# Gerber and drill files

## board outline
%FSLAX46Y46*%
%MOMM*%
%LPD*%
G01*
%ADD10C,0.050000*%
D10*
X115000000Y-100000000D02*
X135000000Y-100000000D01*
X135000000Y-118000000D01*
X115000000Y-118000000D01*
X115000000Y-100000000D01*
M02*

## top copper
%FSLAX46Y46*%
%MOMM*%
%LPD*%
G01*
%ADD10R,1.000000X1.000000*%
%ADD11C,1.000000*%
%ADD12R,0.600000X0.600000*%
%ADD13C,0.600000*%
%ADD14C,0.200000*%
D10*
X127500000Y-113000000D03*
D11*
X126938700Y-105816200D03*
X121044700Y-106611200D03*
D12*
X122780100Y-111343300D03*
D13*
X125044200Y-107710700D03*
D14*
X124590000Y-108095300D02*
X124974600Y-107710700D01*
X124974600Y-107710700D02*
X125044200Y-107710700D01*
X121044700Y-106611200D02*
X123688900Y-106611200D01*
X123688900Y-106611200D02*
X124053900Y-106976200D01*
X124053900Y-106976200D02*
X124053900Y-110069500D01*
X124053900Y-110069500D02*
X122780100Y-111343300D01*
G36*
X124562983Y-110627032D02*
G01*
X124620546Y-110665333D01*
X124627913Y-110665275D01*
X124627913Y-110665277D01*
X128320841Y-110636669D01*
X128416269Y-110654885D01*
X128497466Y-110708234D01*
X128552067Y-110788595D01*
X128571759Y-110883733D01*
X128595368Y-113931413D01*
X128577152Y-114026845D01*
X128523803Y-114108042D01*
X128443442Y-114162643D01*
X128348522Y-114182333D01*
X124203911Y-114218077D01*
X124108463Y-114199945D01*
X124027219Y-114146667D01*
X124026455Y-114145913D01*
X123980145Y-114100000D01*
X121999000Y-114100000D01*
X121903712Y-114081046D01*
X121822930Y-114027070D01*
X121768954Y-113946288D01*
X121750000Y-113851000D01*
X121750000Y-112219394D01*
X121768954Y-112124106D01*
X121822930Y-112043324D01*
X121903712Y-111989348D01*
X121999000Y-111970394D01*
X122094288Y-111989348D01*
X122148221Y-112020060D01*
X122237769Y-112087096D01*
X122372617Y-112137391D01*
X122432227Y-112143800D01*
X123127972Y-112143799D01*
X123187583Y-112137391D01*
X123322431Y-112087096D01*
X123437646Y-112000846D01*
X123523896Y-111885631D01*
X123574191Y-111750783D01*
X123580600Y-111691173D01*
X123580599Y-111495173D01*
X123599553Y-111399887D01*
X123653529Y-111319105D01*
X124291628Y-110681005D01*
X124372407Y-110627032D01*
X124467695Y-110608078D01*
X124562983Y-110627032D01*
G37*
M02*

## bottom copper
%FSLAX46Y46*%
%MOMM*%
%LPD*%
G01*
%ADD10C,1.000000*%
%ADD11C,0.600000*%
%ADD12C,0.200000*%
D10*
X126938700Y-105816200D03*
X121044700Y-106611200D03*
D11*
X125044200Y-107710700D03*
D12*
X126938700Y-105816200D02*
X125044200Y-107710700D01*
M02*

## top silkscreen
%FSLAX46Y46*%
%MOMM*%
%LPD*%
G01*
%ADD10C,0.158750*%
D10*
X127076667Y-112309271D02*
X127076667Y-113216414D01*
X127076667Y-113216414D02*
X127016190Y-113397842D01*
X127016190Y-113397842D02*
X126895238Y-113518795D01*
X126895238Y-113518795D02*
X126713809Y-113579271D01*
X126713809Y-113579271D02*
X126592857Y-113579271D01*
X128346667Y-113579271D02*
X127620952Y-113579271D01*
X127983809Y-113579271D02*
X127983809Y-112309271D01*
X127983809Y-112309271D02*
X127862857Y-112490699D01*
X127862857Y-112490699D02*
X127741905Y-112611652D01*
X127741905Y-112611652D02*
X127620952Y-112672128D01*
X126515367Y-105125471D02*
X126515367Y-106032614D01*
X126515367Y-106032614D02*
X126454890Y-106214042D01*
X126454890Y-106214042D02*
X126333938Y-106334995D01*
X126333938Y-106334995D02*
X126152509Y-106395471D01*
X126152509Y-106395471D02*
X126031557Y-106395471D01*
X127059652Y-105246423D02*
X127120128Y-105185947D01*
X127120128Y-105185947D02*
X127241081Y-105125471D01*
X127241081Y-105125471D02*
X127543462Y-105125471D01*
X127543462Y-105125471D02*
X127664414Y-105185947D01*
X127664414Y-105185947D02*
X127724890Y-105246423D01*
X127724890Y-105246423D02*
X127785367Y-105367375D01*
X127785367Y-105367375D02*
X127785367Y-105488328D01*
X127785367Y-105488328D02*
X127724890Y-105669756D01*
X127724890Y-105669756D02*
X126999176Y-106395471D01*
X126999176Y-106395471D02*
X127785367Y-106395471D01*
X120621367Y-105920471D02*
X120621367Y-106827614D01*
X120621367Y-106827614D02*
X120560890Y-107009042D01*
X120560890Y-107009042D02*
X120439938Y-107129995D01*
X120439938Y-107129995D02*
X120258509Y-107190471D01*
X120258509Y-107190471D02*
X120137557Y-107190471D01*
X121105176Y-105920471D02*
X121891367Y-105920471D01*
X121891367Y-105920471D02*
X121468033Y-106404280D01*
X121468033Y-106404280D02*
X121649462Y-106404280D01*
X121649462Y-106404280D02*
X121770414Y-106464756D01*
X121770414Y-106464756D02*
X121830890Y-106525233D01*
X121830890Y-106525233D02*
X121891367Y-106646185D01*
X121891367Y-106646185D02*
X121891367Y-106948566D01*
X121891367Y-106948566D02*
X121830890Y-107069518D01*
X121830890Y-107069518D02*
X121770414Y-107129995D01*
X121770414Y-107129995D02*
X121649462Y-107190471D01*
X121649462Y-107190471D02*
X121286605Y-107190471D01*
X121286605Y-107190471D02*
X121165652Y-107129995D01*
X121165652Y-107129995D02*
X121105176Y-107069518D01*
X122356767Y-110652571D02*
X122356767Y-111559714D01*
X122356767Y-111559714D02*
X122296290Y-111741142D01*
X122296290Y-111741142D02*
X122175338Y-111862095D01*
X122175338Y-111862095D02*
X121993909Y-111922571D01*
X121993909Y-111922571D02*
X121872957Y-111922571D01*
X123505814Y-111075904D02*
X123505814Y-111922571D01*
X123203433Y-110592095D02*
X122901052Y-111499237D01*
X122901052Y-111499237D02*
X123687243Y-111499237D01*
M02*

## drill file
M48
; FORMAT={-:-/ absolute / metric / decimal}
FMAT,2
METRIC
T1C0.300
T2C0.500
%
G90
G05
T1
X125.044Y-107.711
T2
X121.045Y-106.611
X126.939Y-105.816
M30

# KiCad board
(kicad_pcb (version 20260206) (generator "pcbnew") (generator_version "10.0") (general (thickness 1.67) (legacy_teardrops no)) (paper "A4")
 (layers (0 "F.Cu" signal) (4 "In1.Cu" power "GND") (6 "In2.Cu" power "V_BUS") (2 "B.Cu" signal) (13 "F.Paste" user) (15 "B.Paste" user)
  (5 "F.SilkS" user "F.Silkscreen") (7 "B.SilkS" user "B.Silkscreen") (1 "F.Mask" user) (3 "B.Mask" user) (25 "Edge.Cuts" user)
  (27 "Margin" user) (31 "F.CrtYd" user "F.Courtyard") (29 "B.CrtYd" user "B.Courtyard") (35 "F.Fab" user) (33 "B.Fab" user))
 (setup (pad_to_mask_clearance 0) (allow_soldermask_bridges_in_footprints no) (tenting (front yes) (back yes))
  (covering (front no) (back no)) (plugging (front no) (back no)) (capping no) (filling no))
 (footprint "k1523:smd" (layer "F.Cu") (at 127.5 113)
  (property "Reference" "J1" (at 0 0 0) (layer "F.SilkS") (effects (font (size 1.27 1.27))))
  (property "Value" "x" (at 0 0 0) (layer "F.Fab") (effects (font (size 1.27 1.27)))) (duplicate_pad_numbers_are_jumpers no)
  (pad "1" smd rect (at 0 0) (size 1 1) (layers "F.Cu" "F.Mask") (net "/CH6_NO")))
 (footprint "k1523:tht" (layer "F.Cu") (at 126.9387 105.8162)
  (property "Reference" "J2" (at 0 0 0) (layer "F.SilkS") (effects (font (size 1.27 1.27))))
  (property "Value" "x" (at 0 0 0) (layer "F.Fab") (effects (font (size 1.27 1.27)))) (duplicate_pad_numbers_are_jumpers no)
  (pad "1" thru_hole circle (at 0 0) (size 1 1) (drill 0.5) (layers "*.Cu" "*.Mask") (remove_unused_layers no) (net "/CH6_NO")))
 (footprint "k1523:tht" (layer "F.Cu") (at 121.0447 106.6112)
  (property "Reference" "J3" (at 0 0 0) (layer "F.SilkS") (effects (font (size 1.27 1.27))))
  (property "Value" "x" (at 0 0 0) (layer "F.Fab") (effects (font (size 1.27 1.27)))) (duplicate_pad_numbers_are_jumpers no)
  (pad "1" thru_hole circle (at 0 0) (size 1 1) (drill 0.5) (layers "*.Cu" "*.Mask") (remove_unused_layers no) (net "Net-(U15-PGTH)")))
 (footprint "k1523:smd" (layer "F.Cu") (at 122.7801 111.3433)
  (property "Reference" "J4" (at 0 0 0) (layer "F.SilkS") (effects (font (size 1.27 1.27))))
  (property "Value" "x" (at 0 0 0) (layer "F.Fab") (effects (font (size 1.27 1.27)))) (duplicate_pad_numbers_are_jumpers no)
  (pad "1" smd rect (at 0 0) (size 0.6 0.6) (layers "F.Cu" "F.Mask") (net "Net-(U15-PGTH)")))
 (gr_rect (start 115 100) (end 135 118) (stroke (width 0.05) (type default)) (fill no) (layer "Edge.Cuts"))
 (segment (start 124.59 108.0953) (end 124.9746 107.7107) (width 0.2) (layer "F.Cu") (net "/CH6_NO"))
 (segment (start 124.9746 107.7107) (end 125.0442 107.7107) (width 0.2) (layer "F.Cu") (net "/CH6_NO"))
 (via (at 125.0442 107.7107) (size 0.6) (drill 0.3) (layers "F.Cu" "B.Cu") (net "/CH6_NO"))
 (segment (start 126.9387 105.8162) (end 125.0442 107.7107) (width 0.2) (layer "B.Cu") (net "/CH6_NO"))
 (segment (start 121.0447 106.6112) (end 123.6889 106.6112) (width 0.2) (layer "F.Cu") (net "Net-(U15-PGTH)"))
 (segment (start 123.6889 106.6112) (end 124.0539 106.9762) (width 0.2) (layer "F.Cu") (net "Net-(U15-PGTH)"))
 (segment (start 124.0539 106.9762) (end 124.0539 110.0695) (width 0.2) (layer "F.Cu") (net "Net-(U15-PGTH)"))
 (segment (start 124.0539 110.0695) (end 122.7801 111.3433) (width 0.2) (layer "F.Cu") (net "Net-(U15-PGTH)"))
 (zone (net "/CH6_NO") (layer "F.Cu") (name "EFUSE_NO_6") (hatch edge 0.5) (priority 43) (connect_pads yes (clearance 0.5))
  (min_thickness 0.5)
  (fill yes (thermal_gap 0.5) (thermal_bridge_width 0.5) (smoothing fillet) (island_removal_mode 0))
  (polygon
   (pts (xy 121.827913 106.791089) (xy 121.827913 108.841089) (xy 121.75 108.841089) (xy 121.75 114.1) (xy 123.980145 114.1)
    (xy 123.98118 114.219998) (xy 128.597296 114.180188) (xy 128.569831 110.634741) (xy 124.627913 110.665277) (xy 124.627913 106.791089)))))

